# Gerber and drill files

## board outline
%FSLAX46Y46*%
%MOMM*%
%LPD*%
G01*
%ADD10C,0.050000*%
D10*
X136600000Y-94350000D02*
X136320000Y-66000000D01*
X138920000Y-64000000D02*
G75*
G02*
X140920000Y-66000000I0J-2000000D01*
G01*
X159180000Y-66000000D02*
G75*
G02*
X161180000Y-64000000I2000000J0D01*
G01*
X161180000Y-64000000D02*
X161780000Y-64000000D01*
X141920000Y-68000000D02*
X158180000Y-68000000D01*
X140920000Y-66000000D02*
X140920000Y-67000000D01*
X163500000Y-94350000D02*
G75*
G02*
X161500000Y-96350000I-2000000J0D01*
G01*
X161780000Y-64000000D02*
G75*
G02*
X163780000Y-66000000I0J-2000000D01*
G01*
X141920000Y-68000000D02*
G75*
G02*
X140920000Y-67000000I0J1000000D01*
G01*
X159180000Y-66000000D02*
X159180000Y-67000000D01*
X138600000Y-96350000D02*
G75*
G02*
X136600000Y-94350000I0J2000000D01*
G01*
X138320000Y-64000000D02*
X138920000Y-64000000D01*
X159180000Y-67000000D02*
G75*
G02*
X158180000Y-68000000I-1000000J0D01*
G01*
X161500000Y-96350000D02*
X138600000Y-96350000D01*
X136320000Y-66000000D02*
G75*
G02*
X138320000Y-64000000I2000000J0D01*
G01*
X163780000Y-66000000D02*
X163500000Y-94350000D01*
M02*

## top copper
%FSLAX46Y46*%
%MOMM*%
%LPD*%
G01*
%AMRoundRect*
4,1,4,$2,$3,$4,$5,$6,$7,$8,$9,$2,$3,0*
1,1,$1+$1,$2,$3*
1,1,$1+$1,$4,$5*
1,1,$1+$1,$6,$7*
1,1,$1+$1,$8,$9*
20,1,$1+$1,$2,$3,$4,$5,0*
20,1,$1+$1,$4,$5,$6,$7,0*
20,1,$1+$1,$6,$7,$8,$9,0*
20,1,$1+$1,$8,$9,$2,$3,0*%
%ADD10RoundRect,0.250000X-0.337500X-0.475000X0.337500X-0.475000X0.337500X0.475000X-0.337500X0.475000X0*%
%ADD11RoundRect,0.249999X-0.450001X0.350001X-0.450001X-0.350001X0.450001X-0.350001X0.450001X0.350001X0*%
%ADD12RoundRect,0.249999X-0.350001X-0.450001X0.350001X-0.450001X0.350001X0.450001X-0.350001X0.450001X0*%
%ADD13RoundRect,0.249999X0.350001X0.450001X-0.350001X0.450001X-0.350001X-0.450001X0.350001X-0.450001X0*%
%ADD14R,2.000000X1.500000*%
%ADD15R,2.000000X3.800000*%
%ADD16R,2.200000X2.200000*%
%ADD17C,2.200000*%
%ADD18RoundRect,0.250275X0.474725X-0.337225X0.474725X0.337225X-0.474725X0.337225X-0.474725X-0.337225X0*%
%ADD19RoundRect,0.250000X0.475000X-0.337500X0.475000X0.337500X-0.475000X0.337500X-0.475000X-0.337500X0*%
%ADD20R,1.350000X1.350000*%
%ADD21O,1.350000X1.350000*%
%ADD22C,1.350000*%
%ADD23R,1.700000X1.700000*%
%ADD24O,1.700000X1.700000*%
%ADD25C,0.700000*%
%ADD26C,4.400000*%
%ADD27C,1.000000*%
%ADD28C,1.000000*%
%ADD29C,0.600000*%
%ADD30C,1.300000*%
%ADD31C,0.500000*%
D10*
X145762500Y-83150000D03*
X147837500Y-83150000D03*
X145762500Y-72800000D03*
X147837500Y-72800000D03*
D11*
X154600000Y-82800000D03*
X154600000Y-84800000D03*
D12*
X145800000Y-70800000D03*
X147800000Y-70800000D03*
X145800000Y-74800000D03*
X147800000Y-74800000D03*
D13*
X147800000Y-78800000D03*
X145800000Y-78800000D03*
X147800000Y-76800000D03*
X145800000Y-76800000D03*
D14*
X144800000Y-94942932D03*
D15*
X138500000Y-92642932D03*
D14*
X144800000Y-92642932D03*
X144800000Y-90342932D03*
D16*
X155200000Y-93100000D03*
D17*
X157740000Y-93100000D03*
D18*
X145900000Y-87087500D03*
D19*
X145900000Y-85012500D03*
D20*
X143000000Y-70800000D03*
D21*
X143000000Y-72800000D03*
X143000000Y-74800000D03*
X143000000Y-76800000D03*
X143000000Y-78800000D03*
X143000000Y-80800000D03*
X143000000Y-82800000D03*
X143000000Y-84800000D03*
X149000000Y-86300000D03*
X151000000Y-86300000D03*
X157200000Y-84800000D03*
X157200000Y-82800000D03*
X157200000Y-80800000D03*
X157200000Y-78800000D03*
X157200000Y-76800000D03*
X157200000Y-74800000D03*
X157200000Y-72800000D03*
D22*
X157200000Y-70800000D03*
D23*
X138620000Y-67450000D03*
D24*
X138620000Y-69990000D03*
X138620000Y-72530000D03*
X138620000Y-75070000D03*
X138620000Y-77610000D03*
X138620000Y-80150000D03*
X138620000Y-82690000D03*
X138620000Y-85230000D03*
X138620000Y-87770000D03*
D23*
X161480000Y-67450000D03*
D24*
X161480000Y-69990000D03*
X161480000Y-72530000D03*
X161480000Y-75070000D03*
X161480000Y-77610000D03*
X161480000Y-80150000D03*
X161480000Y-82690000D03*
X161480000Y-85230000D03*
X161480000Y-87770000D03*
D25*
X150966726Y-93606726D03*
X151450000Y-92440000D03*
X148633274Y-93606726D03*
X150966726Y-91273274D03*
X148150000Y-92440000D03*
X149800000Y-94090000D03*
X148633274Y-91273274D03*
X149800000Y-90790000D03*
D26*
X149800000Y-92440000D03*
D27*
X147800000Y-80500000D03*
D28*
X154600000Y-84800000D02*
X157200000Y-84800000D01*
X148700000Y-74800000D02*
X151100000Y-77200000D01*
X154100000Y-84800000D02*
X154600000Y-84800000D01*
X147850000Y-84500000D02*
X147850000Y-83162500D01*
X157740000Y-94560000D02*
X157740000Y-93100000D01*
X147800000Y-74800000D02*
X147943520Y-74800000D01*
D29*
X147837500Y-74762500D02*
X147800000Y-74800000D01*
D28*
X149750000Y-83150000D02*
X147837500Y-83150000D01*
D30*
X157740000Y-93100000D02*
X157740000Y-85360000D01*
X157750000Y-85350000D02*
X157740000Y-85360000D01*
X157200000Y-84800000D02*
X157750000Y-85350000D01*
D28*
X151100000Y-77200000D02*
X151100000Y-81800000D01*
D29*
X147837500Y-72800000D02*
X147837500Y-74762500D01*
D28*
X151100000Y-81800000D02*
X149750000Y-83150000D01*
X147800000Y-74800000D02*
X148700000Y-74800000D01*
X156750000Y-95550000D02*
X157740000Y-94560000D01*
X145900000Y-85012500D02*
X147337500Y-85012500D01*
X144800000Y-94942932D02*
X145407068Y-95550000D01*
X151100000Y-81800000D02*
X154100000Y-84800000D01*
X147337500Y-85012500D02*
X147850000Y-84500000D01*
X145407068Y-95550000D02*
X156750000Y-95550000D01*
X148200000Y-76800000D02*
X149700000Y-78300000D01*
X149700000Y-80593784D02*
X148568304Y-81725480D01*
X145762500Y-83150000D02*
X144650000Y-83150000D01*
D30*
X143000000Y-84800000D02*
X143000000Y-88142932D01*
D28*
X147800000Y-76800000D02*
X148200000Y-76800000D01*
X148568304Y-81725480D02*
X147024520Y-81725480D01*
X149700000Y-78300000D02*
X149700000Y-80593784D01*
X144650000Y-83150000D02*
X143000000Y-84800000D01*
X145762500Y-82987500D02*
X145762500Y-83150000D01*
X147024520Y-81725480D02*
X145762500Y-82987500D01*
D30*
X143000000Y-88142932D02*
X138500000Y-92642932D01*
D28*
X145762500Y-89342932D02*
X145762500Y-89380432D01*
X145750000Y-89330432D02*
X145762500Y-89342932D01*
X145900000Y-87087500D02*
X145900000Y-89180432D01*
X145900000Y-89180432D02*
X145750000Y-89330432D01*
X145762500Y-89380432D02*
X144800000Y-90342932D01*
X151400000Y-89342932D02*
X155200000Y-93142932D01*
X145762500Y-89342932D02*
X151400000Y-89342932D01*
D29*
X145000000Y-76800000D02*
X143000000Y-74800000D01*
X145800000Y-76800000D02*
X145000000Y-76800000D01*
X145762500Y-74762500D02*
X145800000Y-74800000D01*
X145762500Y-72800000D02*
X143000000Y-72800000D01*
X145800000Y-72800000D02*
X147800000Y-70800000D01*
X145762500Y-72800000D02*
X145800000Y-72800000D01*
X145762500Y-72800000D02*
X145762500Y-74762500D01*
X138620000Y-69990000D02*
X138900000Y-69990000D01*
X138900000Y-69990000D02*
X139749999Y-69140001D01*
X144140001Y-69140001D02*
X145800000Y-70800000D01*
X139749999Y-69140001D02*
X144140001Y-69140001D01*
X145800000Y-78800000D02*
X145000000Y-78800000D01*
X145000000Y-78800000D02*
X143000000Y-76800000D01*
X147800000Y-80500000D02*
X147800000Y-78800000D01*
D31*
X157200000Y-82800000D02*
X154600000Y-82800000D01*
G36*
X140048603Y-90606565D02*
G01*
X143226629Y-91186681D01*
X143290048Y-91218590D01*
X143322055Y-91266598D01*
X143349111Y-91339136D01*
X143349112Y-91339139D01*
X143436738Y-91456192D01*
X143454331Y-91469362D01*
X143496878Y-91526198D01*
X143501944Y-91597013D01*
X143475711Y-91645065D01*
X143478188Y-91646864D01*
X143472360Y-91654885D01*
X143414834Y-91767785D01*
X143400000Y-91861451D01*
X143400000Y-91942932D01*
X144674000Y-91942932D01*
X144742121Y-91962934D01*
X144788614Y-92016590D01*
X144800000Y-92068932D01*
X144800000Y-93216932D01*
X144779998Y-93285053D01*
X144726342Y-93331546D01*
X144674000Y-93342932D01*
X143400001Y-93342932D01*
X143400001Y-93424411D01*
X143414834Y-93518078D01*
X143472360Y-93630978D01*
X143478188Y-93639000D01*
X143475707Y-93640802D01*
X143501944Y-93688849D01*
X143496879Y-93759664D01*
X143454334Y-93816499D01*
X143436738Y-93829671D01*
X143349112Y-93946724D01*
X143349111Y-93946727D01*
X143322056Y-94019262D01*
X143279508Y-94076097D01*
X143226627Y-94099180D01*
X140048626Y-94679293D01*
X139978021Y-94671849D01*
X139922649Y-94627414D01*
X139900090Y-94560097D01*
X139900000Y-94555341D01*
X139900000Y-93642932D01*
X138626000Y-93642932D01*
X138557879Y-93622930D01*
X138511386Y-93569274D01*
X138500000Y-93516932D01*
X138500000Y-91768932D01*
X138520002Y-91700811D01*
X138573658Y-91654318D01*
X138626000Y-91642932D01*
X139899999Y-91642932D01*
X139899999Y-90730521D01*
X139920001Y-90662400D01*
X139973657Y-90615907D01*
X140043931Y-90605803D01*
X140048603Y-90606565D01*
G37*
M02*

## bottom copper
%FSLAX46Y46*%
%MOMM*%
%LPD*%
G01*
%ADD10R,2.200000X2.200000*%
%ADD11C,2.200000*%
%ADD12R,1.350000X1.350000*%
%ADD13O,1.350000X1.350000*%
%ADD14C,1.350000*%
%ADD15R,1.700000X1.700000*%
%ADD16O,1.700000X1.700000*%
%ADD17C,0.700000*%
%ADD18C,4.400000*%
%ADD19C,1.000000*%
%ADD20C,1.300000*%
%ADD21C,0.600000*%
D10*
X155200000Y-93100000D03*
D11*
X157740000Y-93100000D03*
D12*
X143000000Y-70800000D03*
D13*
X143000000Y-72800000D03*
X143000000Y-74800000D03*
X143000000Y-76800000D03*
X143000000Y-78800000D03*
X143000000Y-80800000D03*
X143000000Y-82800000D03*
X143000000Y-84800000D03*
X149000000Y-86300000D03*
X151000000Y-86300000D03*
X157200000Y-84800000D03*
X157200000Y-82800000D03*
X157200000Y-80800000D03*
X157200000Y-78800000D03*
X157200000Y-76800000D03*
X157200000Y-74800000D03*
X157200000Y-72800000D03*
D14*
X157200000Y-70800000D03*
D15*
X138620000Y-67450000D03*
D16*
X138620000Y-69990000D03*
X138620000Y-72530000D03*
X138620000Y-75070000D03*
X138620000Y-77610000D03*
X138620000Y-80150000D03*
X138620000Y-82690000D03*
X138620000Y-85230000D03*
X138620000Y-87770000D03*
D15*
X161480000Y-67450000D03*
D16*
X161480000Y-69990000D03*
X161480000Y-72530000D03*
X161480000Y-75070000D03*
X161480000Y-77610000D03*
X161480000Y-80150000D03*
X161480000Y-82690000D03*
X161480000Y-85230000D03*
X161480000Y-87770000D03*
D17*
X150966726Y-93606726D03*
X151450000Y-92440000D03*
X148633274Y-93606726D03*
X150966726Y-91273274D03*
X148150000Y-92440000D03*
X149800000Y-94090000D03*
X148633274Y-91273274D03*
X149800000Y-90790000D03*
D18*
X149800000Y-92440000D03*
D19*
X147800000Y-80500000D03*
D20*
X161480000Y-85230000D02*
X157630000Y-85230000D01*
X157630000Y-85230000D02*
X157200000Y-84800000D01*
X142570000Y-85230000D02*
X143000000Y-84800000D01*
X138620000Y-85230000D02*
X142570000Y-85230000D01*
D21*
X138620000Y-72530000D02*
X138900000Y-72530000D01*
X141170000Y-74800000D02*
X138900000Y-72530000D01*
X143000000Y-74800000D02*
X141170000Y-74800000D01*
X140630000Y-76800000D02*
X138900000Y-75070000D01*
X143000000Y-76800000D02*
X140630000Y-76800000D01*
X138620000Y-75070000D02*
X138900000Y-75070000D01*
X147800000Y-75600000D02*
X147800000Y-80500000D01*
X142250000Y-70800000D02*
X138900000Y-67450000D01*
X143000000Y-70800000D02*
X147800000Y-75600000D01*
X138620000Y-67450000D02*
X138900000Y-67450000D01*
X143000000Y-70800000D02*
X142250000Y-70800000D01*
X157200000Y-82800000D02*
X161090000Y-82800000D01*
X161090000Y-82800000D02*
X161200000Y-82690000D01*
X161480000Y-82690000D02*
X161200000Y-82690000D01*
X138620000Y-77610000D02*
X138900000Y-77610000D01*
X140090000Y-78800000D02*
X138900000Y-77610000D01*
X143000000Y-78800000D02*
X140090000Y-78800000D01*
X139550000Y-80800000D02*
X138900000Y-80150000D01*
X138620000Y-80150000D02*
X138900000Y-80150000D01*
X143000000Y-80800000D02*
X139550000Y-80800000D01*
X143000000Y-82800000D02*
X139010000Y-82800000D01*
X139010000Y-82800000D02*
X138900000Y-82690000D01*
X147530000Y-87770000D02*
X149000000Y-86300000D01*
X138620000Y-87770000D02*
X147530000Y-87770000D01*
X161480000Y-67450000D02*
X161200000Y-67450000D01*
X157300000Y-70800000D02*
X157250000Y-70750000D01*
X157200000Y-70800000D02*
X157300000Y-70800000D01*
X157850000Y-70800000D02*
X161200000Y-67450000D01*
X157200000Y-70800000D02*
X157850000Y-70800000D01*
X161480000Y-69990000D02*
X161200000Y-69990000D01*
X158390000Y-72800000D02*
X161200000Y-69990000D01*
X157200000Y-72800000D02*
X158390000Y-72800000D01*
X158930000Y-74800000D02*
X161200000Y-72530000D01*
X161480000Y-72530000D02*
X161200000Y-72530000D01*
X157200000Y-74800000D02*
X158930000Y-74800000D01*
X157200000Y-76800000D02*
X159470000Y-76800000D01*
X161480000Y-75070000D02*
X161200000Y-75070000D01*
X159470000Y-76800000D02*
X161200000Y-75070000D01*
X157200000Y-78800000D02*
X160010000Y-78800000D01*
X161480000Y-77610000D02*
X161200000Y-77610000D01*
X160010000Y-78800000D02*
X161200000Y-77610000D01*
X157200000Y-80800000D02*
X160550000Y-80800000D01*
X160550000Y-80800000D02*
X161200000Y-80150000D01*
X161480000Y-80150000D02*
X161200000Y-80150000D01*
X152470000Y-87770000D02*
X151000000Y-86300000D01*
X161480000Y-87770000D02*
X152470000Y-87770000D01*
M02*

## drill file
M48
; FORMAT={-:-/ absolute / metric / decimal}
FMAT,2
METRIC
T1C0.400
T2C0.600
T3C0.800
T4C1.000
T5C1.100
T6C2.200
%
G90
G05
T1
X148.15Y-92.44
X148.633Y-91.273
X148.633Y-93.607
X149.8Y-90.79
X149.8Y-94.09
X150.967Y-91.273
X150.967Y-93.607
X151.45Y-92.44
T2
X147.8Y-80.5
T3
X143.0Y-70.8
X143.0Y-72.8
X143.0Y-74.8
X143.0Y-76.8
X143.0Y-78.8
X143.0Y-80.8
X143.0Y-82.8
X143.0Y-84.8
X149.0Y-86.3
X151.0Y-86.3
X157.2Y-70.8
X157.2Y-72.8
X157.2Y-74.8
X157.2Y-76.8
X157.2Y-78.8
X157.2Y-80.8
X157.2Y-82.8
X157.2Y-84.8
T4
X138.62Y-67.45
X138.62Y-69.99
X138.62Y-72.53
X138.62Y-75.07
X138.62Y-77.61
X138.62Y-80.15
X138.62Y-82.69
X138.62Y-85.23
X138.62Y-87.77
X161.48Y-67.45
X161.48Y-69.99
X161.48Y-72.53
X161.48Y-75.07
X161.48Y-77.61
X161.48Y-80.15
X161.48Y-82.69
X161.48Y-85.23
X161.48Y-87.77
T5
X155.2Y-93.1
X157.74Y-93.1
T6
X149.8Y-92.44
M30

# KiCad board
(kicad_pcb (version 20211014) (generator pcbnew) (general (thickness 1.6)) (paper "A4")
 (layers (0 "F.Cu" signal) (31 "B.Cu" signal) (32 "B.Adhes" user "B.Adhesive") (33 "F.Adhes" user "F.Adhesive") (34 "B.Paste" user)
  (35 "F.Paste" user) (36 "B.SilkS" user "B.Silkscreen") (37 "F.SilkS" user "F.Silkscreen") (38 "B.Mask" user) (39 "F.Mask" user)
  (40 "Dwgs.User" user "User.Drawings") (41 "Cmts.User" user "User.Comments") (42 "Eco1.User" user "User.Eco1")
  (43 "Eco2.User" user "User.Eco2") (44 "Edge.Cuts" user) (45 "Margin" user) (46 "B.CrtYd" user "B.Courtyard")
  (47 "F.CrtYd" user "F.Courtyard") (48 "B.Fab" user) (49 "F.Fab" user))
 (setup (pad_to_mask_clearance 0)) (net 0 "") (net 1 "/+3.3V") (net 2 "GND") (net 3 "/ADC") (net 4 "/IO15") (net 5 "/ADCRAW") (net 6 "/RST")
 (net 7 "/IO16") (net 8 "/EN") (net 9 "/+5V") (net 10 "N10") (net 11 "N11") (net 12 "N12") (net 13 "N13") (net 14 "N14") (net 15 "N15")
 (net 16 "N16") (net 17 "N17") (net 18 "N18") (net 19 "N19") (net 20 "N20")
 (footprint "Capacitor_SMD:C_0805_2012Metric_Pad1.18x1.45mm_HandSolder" (layer "F.Cu") (at 146.8 83.15)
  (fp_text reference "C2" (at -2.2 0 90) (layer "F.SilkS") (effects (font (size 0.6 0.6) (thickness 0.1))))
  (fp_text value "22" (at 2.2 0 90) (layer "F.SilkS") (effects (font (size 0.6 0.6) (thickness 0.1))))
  (pad "1" smd roundrect locked (at -1.0375 0) (size 1.175 1.45) (layers "F.Cu" "F.Paste" "F.Mask") (roundrect_rratio 0.2127659574)
   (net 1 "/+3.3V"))
  (pad "2" smd roundrect locked (at 1.0375 0) (size 1.175 1.45) (layers "F.Cu" "F.Paste" "F.Mask") (roundrect_rratio 0.2127659574)
   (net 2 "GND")))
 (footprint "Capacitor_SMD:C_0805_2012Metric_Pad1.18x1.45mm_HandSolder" (layer "F.Cu") (at 146.8 72.8)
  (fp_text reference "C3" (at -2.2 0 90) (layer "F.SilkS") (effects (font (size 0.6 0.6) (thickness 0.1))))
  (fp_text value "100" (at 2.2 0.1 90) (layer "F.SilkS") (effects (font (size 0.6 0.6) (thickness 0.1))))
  (pad "1" smd roundrect locked (at -1.0375 0) (size 1.175 1.45) (layers "F.Cu" "F.Paste" "F.Mask") (roundrect_rratio 0.2127659574)
   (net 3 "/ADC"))
  (pad "2" smd roundrect locked (at 1.0375 0) (size 1.175 1.45) (layers "F.Cu" "F.Paste" "F.Mask") (roundrect_rratio 0.2127659574)
   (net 2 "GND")))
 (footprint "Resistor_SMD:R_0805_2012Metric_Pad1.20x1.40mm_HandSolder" (layer "F.Cu") (at 154.6 83.8 -90)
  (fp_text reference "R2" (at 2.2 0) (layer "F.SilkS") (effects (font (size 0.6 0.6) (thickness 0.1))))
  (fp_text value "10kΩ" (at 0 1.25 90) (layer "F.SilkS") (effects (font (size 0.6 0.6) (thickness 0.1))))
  (pad "1" smd roundrect locked (at -1 0 270) (size 1.2 1.4) (layers "F.Cu" "F.Paste" "F.Mask") (roundrect_rratio 0.2083325) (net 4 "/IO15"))
  (pad "2" smd roundrect locked (at 1 0 270) (size 1.2 1.4) (layers "F.Cu" "F.Paste" "F.Mask") (roundrect_rratio 0.2083325) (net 2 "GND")))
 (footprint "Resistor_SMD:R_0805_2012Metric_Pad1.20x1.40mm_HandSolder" (layer "F.Cu") (at 146.8 70.8)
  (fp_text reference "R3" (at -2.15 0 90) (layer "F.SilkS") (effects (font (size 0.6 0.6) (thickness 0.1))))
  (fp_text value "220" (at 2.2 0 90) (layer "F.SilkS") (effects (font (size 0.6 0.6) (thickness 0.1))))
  (pad "1" smd roundrect locked (at -1 0) (size 1.2 1.4) (layers "F.Cu" "F.Paste" "F.Mask") (roundrect_rratio 0.2083325) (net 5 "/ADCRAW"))
  (pad "2" smd roundrect locked (at 1 0) (size 1.2 1.4) (layers "F.Cu" "F.Paste" "F.Mask") (roundrect_rratio 0.2083325) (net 3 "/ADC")))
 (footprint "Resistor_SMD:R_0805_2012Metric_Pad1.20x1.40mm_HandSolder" (layer "F.Cu") (at 146.8 74.8)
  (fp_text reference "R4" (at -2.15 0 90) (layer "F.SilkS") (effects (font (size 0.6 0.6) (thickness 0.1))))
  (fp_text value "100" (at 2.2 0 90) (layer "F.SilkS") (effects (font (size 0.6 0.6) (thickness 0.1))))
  (pad "1" smd roundrect locked (at -1 0) (size 1.2 1.4) (layers "F.Cu" "F.Paste" "F.Mask") (roundrect_rratio 0.2083325) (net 3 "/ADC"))
  (pad "2" smd roundrect locked (at 1 0) (size 1.2 1.4) (layers "F.Cu" "F.Paste" "F.Mask") (roundrect_rratio 0.2083325) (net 2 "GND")))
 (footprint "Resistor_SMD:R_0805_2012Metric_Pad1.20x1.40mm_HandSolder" (layer "F.Cu") (at 146.8 78.8 180)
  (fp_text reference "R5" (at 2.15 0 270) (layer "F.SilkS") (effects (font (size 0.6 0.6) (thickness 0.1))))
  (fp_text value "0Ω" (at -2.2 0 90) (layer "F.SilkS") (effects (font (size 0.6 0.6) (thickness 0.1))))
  (pad "1" smd roundrect locked (at -1 0 180) (size 1.2 1.4) (layers "F.Cu" "F.Paste" "F.Mask") (roundrect_rratio 0.2083325) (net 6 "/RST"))
  (pad "2" smd roundrect locked (at 1 0 180) (size 1.2 1.4) (layers "F.Cu" "F.Paste" "F.Mask") (roundrect_rratio 0.2083325) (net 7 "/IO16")))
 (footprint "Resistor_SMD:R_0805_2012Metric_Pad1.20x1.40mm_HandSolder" (layer "F.Cu") (at 146.8 76.8 180)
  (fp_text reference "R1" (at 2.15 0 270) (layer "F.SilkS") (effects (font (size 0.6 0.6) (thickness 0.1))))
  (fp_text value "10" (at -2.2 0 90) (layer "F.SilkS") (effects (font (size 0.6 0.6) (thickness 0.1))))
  (pad "1" smd roundrect locked (at -1 0 180) (size 1.2 1.4) (layers "F.Cu" "F.Paste" "F.Mask") (roundrect_rratio 0.2083325)
   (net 1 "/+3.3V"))
  (pad "2" smd roundrect locked (at 1 0 180) (size 1.2 1.4) (layers "F.Cu" "F.Paste" "F.Mask") (roundrect_rratio 0.2083325) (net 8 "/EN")))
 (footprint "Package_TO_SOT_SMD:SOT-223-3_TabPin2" (layer "F.Cu") (at 141.65 92.642932 180)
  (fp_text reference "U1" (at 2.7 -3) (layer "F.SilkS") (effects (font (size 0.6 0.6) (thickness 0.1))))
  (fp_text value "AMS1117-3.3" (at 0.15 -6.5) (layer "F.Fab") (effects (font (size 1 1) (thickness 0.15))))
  (pad "1" smd rect locked (at -3.15 -2.3 180) (size 2 1.5) (layers "F.Cu" "F.Paste" "F.Mask") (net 2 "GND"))
  (pad "2" smd rect locked (at 3.15 0 180) (size 2 3.8) (layers "F.Cu" "F.Paste" "F.Mask") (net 1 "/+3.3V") (zone_connect 1)
   (thermal_width 3.3) (thermal_gap 0.4))
  (pad "2" smd rect locked (at -3.15 0 180) (size 2 1.5) (layers "F.Cu" "F.Paste" "F.Mask") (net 1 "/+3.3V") (zone_connect 1)
   (thermal_width 1.4) (thermal_gap 0.4))
  (pad "3" smd rect locked (at -3.15 2.3 180) (size 2 1.5) (layers "F.Cu" "F.Paste" "F.Mask") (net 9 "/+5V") (zone_connect 1)
   (thermal_width 1) (thermal_gap 0.5)))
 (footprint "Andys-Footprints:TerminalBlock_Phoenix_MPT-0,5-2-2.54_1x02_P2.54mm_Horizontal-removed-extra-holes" (layer "F.Cu")
  (at 155.2 93.1)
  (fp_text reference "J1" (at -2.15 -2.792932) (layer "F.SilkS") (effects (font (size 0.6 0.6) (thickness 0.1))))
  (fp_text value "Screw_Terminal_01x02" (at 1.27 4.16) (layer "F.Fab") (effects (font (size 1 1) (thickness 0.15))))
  (pad "1" thru_hole rect locked (at 0 0) (size 2.2 2.2) (drill 1.1) (layers *.Cu *.Mask) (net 9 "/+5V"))
  (pad "2" thru_hole circle locked (at 2.54 0) (size 2.2 2.2) (drill 1.1) (layers *.Cu *.Mask) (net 2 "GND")))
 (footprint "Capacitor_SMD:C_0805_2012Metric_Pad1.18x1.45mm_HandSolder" (layer "F.Cu") (at 145.9 86.05 90)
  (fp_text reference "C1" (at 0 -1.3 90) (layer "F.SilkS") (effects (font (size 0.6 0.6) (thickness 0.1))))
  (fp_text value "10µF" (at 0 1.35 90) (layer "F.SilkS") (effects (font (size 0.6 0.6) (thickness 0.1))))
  (pad "1" smd roundrect locked (at -1.0375 0 90) (size 1.175 1.45) (layers "F.Cu" "F.Paste" "F.Mask") (roundrect_rratio 0.213)
   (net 9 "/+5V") (zone_connect 1) (thermal_width 1) (thermal_gap 0.5))
  (pad "2" smd roundrect locked (at 1.0375 0 90) (size 1.175 1.45) (layers "F.Cu" "F.Paste" "F.Mask") (roundrect_rratio 0.2127659574)
   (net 2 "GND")))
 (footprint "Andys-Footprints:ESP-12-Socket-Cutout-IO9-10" (layer "F.Cu") (at 143 70.8)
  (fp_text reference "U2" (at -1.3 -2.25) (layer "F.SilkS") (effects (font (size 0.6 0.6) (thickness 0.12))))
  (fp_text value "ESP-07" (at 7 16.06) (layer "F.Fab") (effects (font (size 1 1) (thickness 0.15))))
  (pad "1" thru_hole rect (at 0 0) (size 1.35 1.35) (drill 0.8) (layers *.Cu *.Mask) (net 6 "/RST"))
  (pad "2" thru_hole oval (at 0 2) (size 1.35 1.35) (drill 0.8) (layers *.Cu *.Mask) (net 3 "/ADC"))
  (pad "3" thru_hole oval (at 0 4) (size 1.35 1.35) (drill 0.8) (layers *.Cu *.Mask) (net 8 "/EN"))
  (pad "4" thru_hole oval (at 0 6) (size 1.35 1.35) (drill 0.8) (layers *.Cu *.Mask) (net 7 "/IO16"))
  (pad "5" thru_hole oval (at 0 8) (size 1.35 1.35) (drill 0.8) (layers *.Cu *.Mask) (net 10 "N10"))
  (pad "6" thru_hole oval (at 0 10) (size 1.35 1.35) (drill 0.8) (layers *.Cu *.Mask) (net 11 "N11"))
  (pad "7" thru_hole oval (at 0 12) (size 1.35 1.35) (drill 0.8) (layers *.Cu *.Mask) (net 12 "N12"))
  (pad "8" thru_hole oval (at 0 14) (size 1.35 1.35) (drill 0.8) (layers *.Cu *.Mask) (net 1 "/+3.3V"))
  (pad "11" thru_hole oval (at 6 15.5 270) (size 1.35 1.35) (drill 0.8) (layers *.Cu *.Mask) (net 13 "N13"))
  (pad "12" thru_hole oval (at 8 15.5 270) (size 1.35 1.35) (drill 0.8) (layers *.Cu *.Mask) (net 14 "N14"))
  (pad "15" thru_hole oval (at 14.2 14) (size 1.35 1.35) (drill 0.8) (layers *.Cu *.Mask) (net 2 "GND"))
  (pad "16" thru_hole oval (at 14.2 12) (size 1.35 1.35) (drill 0.8) (layers *.Cu *.Mask) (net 4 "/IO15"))
  (pad "17" thru_hole oval (at 14.2 10) (size 1.35 1.35) (drill 0.8) (layers *.Cu *.Mask) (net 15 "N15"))
  (pad "18" thru_hole oval (at 14.2 8) (size 1.35 1.35) (drill 0.8) (layers *.Cu *.Mask) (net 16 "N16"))
  (pad "19" thru_hole oval (at 14.2 6) (size 1.35 1.35) (drill 0.8) (layers *.Cu *.Mask) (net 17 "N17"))
  (pad "20" thru_hole oval (at 14.2 4) (size 1.35 1.35) (drill 0.8) (layers *.Cu *.Mask) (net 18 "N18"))
  (pad "21" thru_hole oval (at 14.2 2) (size 1.35 1.35) (drill 0.8) (layers *.Cu *.Mask) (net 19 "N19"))
  (pad "22" thru_hole circle (at 14.2 0) (size 1.35 1.35) (drill 0.8) (layers *.Cu *.Mask) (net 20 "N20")))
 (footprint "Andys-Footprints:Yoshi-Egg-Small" (layer "F.Cu") (at 161.45 92.35)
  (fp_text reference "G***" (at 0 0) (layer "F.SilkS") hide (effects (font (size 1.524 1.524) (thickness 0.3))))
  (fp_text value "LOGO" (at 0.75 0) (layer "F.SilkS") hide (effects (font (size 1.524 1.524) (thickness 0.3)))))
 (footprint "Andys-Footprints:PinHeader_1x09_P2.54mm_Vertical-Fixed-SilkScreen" (layer "F.Cu") (at 138.62 67.45)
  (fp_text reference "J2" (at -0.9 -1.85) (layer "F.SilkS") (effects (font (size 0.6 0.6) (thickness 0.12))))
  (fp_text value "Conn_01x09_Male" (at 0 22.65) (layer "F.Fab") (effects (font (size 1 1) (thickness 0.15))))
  (pad "1" thru_hole rect (at 0 0) (size 1.7 1.7) (drill 1) (layers *.Cu *.Mask) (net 6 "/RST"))
  (pad "2" thru_hole oval (at 0 2.54) (size 1.7 1.7) (drill 1) (layers *.Cu *.Mask) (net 5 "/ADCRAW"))
  (pad "3" thru_hole oval (at 0 5.08) (size 1.7 1.7) (drill 1) (layers *.Cu *.Mask) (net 8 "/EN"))
  (pad "4" thru_hole oval (at 0 7.62) (size 1.7 1.7) (drill 1) (layers *.Cu *.Mask) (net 7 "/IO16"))
  (pad "5" thru_hole oval (at 0 10.16) (size 1.7 1.7) (drill 1) (layers *.Cu *.Mask) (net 10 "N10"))
  (pad "6" thru_hole oval (at 0 12.7) (size 1.7 1.7) (drill 1) (layers *.Cu *.Mask) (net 11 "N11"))
  (pad "7" thru_hole oval (at 0 15.24) (size 1.7 1.7) (drill 1) (layers *.Cu *.Mask) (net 12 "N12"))
  (pad "8" thru_hole oval (at 0 17.78) (size 1.7 1.7) (drill 1) (layers *.Cu *.Mask) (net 1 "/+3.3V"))
  (pad "9" thru_hole oval (at 0 20.32) (size 1.7 1.7) (drill 1) (layers *.Cu *.Mask) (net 13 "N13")))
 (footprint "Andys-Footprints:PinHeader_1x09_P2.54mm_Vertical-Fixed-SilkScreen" (layer "F.Cu") (at 161.48 67.45)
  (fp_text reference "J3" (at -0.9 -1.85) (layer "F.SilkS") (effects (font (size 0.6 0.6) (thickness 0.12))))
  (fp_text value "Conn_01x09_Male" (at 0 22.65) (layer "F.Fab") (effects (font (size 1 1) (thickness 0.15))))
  (pad "1" thru_hole rect (at 0 0) (size 1.7 1.7) (drill 1) (layers *.Cu *.Mask) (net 20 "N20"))
  (pad "2" thru_hole oval (at 0 2.54) (size 1.7 1.7) (drill 1) (layers *.Cu *.Mask) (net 19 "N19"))
  (pad "3" thru_hole oval (at 0 5.08) (size 1.7 1.7) (drill 1) (layers *.Cu *.Mask) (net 18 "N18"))
  (pad "4" thru_hole oval (at 0 7.62) (size 1.7 1.7) (drill 1) (layers *.Cu *.Mask) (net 17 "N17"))
  (pad "5" thru_hole oval (at 0 10.16) (size 1.7 1.7) (drill 1) (layers *.Cu *.Mask) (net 16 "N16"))
  (pad "6" thru_hole oval (at 0 12.7) (size 1.7 1.7) (drill 1) (layers *.Cu *.Mask) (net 15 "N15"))
  (pad "7" thru_hole oval (at 0 15.24) (size 1.7 1.7) (drill 1) (layers *.Cu *.Mask) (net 4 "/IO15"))
  (pad "8" thru_hole oval (at 0 17.78) (size 1.7 1.7) (drill 1) (layers *.Cu *.Mask) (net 2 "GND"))
  (pad "9" thru_hole oval (at 0 20.32) (size 1.7 1.7) (drill 1) (layers *.Cu *.Mask) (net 14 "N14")))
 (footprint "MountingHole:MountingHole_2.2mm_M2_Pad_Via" (layer "F.Cu") (at 149.8 92.44)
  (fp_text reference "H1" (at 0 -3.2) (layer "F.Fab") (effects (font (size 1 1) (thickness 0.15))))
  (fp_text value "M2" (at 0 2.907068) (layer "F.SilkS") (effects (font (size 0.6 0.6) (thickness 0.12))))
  (pad "1" thru_hole circle locked (at 1.166726 1.166726) (size 0.7 0.7) (drill 0.4) (layers *.Cu *.Mask))
  (pad "1" thru_hole circle locked (at 1.65 0) (size 0.7 0.7) (drill 0.4) (layers *.Cu *.Mask))
  (pad "1" thru_hole circle locked (at -1.166726 1.166726) (size 0.7 0.7) (drill 0.4) (layers *.Cu *.Mask))
  (pad "1" thru_hole circle locked (at 1.166726 -1.166726) (size 0.7 0.7) (drill 0.4) (layers *.Cu *.Mask))
  (pad "1" thru_hole circle locked (at -1.65 0) (size 0.7 0.7) (drill 0.4) (layers *.Cu *.Mask))
  (pad "1" thru_hole circle locked (at 0 1.65) (size 0.7 0.7) (drill 0.4) (layers *.Cu *.Mask))
  (pad "1" thru_hole circle locked (at -1.166726 -1.166726) (size 0.7 0.7) (drill 0.4) (layers *.Cu *.Mask))
  (pad "1" thru_hole circle locked (at 0 -1.65) (size 0.7 0.7) (drill 0.4) (layers *.Cu *.Mask))
  (pad "1" thru_hole circle locked (at 0 0) (size 4.4 4.4) (drill 2.2) (layers *.Cu *.Mask)))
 (gr_line (start 136.6 94.35) (end 136.32 66) (layer "Edge.Cuts") (width 0.05))
 (gr_arc (start 138.92 64) (mid 140.334214 64.585786) (end 140.92 66) (layer "Edge.Cuts") (width 0.05))
 (gr_arc (start 159.18 66) (mid 159.765786 64.585786) (end 161.18 64) (layer "Edge.Cuts") (width 0.05))
 (gr_line (start 161.18 64) (end 161.78 64) (layer "Edge.Cuts") (width 0.05))
 (gr_line (start 141.92 68) (end 158.18 68) (layer "Edge.Cuts") (width 0.05))
 (gr_line (start 140.92 66) (end 140.92 67) (layer "Edge.Cuts") (width 0.05))
 (gr_arc (start 163.5 94.35) (mid 162.914214 95.764214) (end 161.5 96.35) (layer "Edge.Cuts") (width 0.05))
 (gr_arc (start 161.78 64) (mid 163.194214 64.585786) (end 163.78 66) (layer "Edge.Cuts") (width 0.05))
 (gr_arc (start 141.92 68) (mid 141.212893 67.707107) (end 140.92 67) (layer "Edge.Cuts") (width 0.05))
 (gr_line (start 159.18 66) (end 159.18 67) (layer "Edge.Cuts") (width 0.05))
 (gr_arc (start 138.6 96.35) (mid 137.185786 95.764214) (end 136.6 94.35) (layer "Edge.Cuts") (width 0.05))
 (gr_line (start 138.32 64) (end 138.92 64) (layer "Edge.Cuts") (width 0.05))
 (gr_arc (start 159.18 67) (mid 158.887107 67.707107) (end 158.18 68) (layer "Edge.Cuts") (width 0.05))
 (gr_line (start 161.5 96.35) (end 138.6 96.35) (layer "Edge.Cuts") (width 0.05))
 (gr_arc (start 136.32 66) (mid 136.905786 64.585786) (end 138.32 64) (layer "Edge.Cuts") (width 0.05))
 (gr_line (start 163.78 66) (end 163.5 94.35) (layer "Edge.Cuts") (width 0.05))
 (segment (start 154.6 84.8) (end 157.2 84.8) (width 1) (layer "F.Cu") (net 2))
 (segment (start 148.7 74.8) (end 151.1 77.2) (width 1) (layer "F.Cu") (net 2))
 (segment (start 154.1 84.8) (end 154.6 84.8) (width 1) (layer "F.Cu") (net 2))
 (segment (start 147.85 84.5) (end 147.85 83.1625) (width 1) (layer "F.Cu") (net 2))
 (segment (start 157.74 94.56) (end 157.74 93.1) (width 1) (layer "F.Cu") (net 2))
 (segment (start 147.8 74.8) (end 147.94352 74.8) (width 1) (layer "F.Cu") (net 2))
 (segment (start 147.8375 74.7625) (end 147.8 74.8) (width 0.6) (layer "F.Cu") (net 2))
 (segment (start 149.75 83.15) (end 147.8375 83.15) (width 1) (layer "F.Cu") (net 2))
 (segment (start 157.74 93.1) (end 157.74 85.36) (width 1.3) (layer "F.Cu") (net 2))
 (segment (start 157.75 85.35) (end 157.74 85.36) (width 1.3) (layer "F.Cu") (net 2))
 (segment (start 157.2 84.8) (end 157.75 85.35) (width 1.3) (layer "F.Cu") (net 2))
 (segment (start 151.1 77.2) (end 151.1 81.8) (width 1) (layer "F.Cu") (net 2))
 (segment (start 147.8375 72.8) (end 147.8375 74.7625) (width 0.6) (layer "F.Cu") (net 2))
 (segment (start 151.1 81.8) (end 149.75 83.15) (width 1) (layer "F.Cu") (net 2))
 (segment (start 147.8 74.8) (end 148.7 74.8) (width 1) (layer "F.Cu") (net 2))
 (segment (start 156.75 95.55) (end 157.74 94.56) (width 1) (layer "F.Cu") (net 2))
 (segment (start 145.9 85.0125) (end 147.3375 85.0125) (width 1) (layer "F.Cu") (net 2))
 (segment (start 144.8 94.942932) (end 145.407068 95.55) (width 1) (layer "F.Cu") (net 2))
 (segment (start 151.1 81.8) (end 154.1 84.8) (width 1) (layer "F.Cu") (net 2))
 (segment (start 147.3375 85.0125) (end 147.85 84.5) (width 1) (layer "F.Cu") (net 2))
 (segment (start 145.407068 95.55) (end 156.75 95.55) (width 1) (layer "F.Cu") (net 2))
 (segment (start 161.48 85.23) (end 157.63 85.23) (width 1.3) (layer "B.Cu") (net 2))
 (segment (start 157.63 85.23) (end 157.2 84.8) (width 1.3) (layer "B.Cu") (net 2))
 (segment (start 148.2 76.8) (end 149.7 78.3) (width 1) (layer "F.Cu") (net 1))
 (segment (start 149.7 80.593784) (end 148.568304 81.72548) (width 1) (layer "F.Cu") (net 1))
 (segment (start 145.7625 83.15) (end 144.65 83.15) (width 1) (layer "F.Cu") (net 1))
 (segment (start 143 84.8) (end 143 88.142932) (width 1.3) (layer "F.Cu") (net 1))
 (segment (start 147.8 76.8) (end 148.2 76.8) (width 1) (layer "F.Cu") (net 1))
 (segment (start 148.568304 81.72548) (end 147.02452 81.72548) (width 1) (layer "F.Cu") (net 1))
 (segment (start 149.7 78.3) (end 149.7 80.593784) (width 1) (layer "F.Cu") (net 1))
 (segment (start 144.65 83.15) (end 143 84.8) (width 1) (layer "F.Cu") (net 1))
 (segment (start 145.7625 82.9875) (end 145.7625 83.15) (width 1) (layer "F.Cu") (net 1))
 (segment (start 147.02452 81.72548) (end 145.7625 82.9875) (width 1) (layer "F.Cu") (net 1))
 (segment (start 143 88.142932) (end 138.5 92.642932) (width 1.3) (layer "F.Cu") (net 1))
 (segment (start 142.57 85.23) (end 143 84.8) (width 1.3) (layer "B.Cu") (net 1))
 (segment (start 138.62 85.23) (end 142.57 85.23) (width 1.3) (layer "B.Cu") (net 1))
 (segment (start 145.7625 89.342932) (end 145.7625 89.380432) (width 1) (layer "F.Cu") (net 9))
 (segment (start 145.75 89.330432) (end 145.7625 89.342932) (width 1) (layer "F.Cu") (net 9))
 (segment (start 145.9 87.0875) (end 145.9 89.180432) (width 1) (layer "F.Cu") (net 9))
 (segment (start 145.9 89.180432) (end 145.75 89.330432) (width 1) (layer "F.Cu") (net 9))
 (segment (start 145.7625 89.380432) (end 144.8 90.342932) (width 1) (layer "F.Cu") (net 9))
 (segment (start 151.4 89.342932) (end 155.2 93.142932) (width 1) (layer "F.Cu") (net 9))
 (segment (start 145.7625 89.342932) (end 151.4 89.342932) (width 1) (layer "F.Cu") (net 9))
 (segment (start 145 76.8) (end 143 74.8) (width 0.6) (layer "F.Cu") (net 8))
 (segment (start 145.8 76.8) (end 145 76.8) (width 0.6) (layer "F.Cu") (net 8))
 (segment (start 138.62 72.53) (end 138.9 72.53) (width 0.6) (layer "B.Cu") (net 8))
 (segment (start 141.17 74.8) (end 138.9 72.53) (width 0.6) (layer "B.Cu") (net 8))
 (segment (start 143 74.8) (end 141.17 74.8) (width 0.6) (layer "B.Cu") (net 8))
 (segment (start 145.7625 74.7625) (end 145.8 74.8) (width 0.6) (layer "F.Cu") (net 3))
 (segment (start 145.7625 72.8) (end 143 72.8) (width 0.6) (layer "F.Cu") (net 3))
 (segment (start 145.8 72.8) (end 147.8 70.8) (width 0.6) (layer "F.Cu") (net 3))
 (segment (start 145.7625 72.8) (end 145.8 72.8) (width 0.6) (layer "F.Cu") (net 3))
 (segment (start 145.7625 72.8) (end 145.7625 74.7625) (width 0.6) (layer "F.Cu") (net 3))
 (segment (start 138.62 69.99) (end 138.9 69.99) (width 0.6) (layer "F.Cu") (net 5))
 (segment (start 138.9 69.99) (end 139.749999 69.140001) (width 0.6) (layer "F.Cu") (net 5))
 (segment (start 144.140001 69.140001) (end 145.8 70.8) (width 0.6) (layer "F.Cu") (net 5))
 (segment (start 139.749999 69.140001) (end 144.140001 69.140001) (width 0.6) (layer "F.Cu") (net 5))
 (segment (start 145.8 78.8) (end 145 78.8) (width 0.6) (layer "F.Cu") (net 7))
 (segment (start 145 78.8) (end 143 76.8) (width 0.6) (layer "F.Cu") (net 7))
 (segment (start 140.63 76.8) (end 138.9 75.07) (width 0.6) (layer "B.Cu") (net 7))
 (segment (start 143 76.8) (end 140.63 76.8) (width 0.6) (layer "B.Cu") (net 7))
 (segment (start 138.62 75.07) (end 138.9 75.07) (width 0.6) (layer "B.Cu") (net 7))
 (segment (start 147.8 80.5) (end 147.8 78.8) (width 0.6) (layer "F.Cu") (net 6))
 (via (at 147.8 80.5) (size 1) (drill 0.6) (layers "F.Cu" "B.Cu") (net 6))
 (segment (start 147.8 75.6) (end 147.8 80.5) (width 0.6) (layer "B.Cu") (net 6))
 (segment (start 142.25 70.8) (end 138.9 67.45) (width 0.6) (layer "B.Cu") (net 6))
 (segment (start 143 70.8) (end 147.8 75.6) (width 0.6) (layer "B.Cu") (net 6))
 (segment (start 138.62 67.45) (end 138.9 67.45) (width 0.6) (layer "B.Cu") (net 6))
 (segment (start 143 70.8) (end 142.25 70.8) (width 0.6) (layer "B.Cu") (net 6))
 (segment (start 157.2 82.8) (end 154.6 82.8) (width 0.5) (layer "F.Cu") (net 4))
 (segment (start 157.2 82.8) (end 161.09 82.8) (width 0.6) (layer "B.Cu") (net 4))
 (segment (start 161.09 82.8) (end 161.2 82.69) (width 0.6) (layer "B.Cu") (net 4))
 (segment (start 161.48 82.69) (end 161.2 82.69) (width 0.6) (layer "B.Cu") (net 4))
 (segment (start 138.62 77.61) (end 138.9 77.61) (width 0.6) (layer "B.Cu") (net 10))
 (segment (start 140.09 78.8) (end 138.9 77.61) (width 0.6) (layer "B.Cu") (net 10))
 (segment (start 143 78.8) (end 140.09 78.8) (width 0.6) (layer "B.Cu") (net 10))
 (segment (start 139.55 80.8) (end 138.9 80.15) (width 0.6) (layer "B.Cu") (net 11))
 (segment (start 138.62 80.15) (end 138.9 80.15) (width 0.6) (layer "B.Cu") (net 11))
 (segment (start 143 80.8) (end 139.55 80.8) (width 0.6) (layer "B.Cu") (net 11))
 (segment (start 143 82.8) (end 139.01 82.8) (width 0.6) (layer "B.Cu") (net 12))
 (segment (start 139.01 82.8) (end 138.9 82.69) (width 0.6) (layer "B.Cu") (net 12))
 (segment (start 147.53 87.77) (end 149 86.3) (width 0.6) (layer "B.Cu") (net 13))
 (segment (start 138.62 87.77) (end 147.53 87.77) (width 0.6) (layer "B.Cu") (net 13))
 (segment (start 161.48 67.45) (end 161.2 67.45) (width 0.6) (layer "B.Cu") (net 20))
 (segment (start 157.3 70.8) (end 157.25 70.75) (width 0.6) (layer "B.Cu") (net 20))
 (segment (start 157.2 70.8) (end 157.3 70.8) (width 0.6) (layer "B.Cu") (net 20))
 (segment (start 157.85 70.8) (end 161.2 67.45) (width 0.6) (layer "B.Cu") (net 20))
 (segment (start 157.2 70.8) (end 157.85 70.8) (width 0.6) (layer "B.Cu") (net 20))
 (segment (start 161.48 69.99) (end 161.2 69.99) (width 0.6) (layer "B.Cu") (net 19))
 (segment (start 158.39 72.8) (end 161.2 69.99) (width 0.6) (layer "B.Cu") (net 19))
 (segment (start 157.2 72.8) (end 158.39 72.8) (width 0.6) (layer "B.Cu") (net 19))
 (segment (start 158.93 74.8) (end 161.2 72.53) (width 0.6) (layer "B.Cu") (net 18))
 (segment (start 161.48 72.53) (end 161.2 72.53) (width 0.6) (layer "B.Cu") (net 18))
 (segment (start 157.2 74.8) (end 158.93 74.8) (width 0.6) (layer "B.Cu") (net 18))
 (segment (start 157.2 76.8) (end 159.47 76.8) (width 0.6) (layer "B.Cu") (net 17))
 (segment (start 161.48 75.07) (end 161.2 75.07) (width 0.6) (layer "B.Cu") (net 17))
 (segment (start 159.47 76.8) (end 161.2 75.07) (width 0.6) (layer "B.Cu") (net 17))
 (segment (start 157.2 78.8) (end 160.01 78.8) (width 0.6) (layer "B.Cu") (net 16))
 (segment (start 161.48 77.61) (end 161.2 77.61) (width 0.6) (layer "B.Cu") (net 16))
 (segment (start 160.01 78.8) (end 161.2 77.61) (width 0.6) (layer "B.Cu") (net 16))
 (segment (start 157.2 80.8) (end 160.55 80.8) (width 0.6) (layer "B.Cu") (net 15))
 (segment (start 160.55 80.8) (end 161.2 80.15) (width 0.6) (layer "B.Cu") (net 15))
 (segment (start 161.48 80.15) (end 161.2 80.15) (width 0.6) (layer "B.Cu") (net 15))
 (segment (start 152.47 87.77) (end 151 86.3) (width 0.6) (layer "B.Cu") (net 14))
 (segment (start 161.48 87.77) (end 152.47 87.77) (width 0.6) (layer "B.Cu") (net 14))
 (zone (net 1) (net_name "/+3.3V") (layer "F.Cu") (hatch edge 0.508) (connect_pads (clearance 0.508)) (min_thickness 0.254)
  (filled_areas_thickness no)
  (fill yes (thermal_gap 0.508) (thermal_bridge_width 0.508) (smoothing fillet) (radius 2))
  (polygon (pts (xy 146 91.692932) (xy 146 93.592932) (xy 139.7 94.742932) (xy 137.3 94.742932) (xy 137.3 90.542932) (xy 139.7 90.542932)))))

